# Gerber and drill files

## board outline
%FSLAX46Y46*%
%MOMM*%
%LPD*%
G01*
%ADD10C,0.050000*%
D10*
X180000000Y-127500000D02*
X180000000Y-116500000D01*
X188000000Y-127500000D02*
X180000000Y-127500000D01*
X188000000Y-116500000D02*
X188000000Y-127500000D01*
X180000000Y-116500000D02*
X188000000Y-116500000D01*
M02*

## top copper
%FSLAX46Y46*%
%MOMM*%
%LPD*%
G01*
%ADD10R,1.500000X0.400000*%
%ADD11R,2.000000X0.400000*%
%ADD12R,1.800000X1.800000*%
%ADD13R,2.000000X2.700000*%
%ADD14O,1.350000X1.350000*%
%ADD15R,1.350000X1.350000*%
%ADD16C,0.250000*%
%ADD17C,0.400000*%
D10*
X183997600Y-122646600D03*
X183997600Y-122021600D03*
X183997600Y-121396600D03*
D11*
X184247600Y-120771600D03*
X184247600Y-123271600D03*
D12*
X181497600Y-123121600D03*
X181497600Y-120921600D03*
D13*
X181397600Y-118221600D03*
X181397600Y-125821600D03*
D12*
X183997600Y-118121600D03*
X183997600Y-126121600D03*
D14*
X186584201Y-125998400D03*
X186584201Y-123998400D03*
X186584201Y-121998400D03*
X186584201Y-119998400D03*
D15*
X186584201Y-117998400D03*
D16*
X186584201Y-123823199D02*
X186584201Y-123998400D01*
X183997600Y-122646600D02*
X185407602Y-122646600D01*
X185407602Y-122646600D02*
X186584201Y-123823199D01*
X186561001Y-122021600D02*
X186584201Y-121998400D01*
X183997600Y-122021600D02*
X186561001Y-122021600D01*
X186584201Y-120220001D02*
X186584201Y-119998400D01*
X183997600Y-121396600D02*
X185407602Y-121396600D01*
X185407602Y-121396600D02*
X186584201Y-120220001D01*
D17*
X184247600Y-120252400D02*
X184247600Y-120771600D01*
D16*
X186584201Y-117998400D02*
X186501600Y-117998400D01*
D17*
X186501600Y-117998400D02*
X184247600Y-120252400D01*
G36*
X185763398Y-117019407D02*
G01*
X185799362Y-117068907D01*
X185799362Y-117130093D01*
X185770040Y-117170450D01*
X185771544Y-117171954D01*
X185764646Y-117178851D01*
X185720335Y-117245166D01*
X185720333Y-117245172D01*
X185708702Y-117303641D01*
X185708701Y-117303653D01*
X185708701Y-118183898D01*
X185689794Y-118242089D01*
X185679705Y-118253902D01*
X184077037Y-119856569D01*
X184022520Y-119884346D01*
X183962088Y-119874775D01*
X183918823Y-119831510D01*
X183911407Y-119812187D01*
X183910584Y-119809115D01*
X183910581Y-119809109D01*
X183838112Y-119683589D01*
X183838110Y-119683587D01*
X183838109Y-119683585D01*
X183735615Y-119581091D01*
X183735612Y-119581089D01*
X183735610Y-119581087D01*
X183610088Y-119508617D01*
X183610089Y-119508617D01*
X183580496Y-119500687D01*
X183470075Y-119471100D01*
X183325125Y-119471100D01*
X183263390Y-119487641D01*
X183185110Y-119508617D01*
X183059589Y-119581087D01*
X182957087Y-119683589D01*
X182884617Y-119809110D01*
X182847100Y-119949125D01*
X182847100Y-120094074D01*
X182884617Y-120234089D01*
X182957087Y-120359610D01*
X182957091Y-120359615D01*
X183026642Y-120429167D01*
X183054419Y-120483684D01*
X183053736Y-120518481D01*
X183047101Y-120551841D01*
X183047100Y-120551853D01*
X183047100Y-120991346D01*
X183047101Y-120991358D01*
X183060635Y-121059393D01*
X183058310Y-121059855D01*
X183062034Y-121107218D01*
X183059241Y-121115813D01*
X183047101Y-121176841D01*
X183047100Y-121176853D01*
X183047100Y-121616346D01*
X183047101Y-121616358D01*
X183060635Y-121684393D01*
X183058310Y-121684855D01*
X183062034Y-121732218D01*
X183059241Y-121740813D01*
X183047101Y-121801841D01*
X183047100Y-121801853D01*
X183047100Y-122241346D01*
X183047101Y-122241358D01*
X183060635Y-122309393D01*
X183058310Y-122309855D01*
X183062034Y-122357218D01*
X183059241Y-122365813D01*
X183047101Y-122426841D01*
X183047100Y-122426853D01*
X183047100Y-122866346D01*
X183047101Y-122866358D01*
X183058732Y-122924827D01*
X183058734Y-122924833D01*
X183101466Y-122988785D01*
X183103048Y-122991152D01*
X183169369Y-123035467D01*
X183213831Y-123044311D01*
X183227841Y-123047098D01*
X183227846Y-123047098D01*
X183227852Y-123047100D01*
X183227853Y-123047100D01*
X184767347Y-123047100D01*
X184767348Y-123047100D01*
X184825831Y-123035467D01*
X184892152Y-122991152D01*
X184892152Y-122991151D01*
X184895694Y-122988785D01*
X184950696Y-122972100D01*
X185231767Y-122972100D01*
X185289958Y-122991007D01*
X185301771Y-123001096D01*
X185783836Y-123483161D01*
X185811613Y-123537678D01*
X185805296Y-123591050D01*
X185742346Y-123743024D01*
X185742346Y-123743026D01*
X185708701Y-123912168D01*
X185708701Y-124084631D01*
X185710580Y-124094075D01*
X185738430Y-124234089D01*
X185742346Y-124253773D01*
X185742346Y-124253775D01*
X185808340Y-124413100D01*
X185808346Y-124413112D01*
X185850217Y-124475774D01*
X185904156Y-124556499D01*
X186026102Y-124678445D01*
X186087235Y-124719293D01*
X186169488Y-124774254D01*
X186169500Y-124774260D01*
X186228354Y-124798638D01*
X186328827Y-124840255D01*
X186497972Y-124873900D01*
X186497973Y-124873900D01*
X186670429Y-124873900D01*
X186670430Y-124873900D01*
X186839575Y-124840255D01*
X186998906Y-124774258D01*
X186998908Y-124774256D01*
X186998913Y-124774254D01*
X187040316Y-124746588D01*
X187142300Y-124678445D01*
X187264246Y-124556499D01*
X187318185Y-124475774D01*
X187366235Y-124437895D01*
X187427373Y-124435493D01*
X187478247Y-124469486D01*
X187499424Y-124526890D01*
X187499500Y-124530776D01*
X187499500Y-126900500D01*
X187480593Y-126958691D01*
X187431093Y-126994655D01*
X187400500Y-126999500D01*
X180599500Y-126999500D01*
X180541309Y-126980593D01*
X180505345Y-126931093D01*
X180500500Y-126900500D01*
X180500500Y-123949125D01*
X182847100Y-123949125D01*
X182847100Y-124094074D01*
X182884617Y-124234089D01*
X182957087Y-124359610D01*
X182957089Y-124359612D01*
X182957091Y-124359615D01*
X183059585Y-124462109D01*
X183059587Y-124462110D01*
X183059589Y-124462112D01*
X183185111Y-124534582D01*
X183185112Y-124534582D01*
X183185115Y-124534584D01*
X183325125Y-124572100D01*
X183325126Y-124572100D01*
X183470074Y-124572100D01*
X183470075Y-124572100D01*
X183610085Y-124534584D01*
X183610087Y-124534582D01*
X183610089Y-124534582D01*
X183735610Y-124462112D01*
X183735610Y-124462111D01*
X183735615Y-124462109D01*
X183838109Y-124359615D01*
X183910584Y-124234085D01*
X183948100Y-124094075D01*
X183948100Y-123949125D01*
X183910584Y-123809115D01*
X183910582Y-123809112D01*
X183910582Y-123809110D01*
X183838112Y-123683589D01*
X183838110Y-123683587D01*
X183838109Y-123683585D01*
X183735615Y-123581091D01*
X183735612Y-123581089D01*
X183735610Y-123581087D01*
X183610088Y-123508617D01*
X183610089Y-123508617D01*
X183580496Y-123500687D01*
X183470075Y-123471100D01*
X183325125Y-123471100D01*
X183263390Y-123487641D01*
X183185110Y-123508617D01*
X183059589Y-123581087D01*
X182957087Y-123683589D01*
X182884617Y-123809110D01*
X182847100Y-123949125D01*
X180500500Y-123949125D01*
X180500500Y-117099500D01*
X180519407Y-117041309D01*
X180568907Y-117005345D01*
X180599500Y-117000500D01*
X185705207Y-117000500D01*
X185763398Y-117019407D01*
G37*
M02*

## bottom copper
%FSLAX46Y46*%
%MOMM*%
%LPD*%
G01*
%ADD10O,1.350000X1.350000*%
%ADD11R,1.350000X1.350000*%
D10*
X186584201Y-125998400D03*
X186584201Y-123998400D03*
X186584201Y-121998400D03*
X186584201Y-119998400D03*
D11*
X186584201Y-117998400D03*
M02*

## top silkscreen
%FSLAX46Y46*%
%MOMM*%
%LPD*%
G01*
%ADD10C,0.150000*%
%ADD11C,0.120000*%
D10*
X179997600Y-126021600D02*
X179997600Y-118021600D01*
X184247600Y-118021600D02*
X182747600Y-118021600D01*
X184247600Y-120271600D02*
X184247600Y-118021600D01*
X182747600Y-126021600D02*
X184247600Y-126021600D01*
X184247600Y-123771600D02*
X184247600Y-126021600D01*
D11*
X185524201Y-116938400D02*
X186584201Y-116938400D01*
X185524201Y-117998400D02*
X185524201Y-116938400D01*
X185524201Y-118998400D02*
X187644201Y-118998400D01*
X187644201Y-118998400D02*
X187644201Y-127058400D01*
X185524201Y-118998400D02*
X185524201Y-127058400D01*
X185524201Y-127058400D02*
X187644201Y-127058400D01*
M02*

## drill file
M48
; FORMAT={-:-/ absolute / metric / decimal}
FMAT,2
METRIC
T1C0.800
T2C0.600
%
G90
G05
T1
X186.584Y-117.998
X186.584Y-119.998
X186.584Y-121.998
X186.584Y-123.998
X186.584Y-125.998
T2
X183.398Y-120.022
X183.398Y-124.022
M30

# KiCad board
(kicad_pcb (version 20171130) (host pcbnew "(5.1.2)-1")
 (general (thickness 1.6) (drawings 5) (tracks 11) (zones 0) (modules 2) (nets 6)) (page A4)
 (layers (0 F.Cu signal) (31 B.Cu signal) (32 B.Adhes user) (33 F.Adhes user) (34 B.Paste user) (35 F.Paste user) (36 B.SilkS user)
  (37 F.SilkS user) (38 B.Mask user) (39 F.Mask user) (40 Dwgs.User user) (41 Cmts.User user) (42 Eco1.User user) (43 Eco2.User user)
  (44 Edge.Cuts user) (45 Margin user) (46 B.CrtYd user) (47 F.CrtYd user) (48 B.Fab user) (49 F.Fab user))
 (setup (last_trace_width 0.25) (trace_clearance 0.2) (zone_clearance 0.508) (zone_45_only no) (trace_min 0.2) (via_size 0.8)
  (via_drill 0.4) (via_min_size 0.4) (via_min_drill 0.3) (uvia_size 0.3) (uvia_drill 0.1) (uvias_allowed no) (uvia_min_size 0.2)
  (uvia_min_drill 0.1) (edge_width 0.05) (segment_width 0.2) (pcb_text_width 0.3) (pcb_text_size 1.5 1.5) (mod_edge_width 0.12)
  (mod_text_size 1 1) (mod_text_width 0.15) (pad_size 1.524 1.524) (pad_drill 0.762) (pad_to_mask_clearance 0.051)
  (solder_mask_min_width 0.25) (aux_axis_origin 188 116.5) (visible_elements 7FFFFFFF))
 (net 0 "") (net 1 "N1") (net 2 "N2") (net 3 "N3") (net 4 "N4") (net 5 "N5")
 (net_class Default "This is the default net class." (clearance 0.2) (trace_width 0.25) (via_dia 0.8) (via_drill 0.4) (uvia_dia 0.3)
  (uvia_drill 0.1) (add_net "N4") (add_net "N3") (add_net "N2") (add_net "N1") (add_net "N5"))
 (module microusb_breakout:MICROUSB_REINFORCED (layer F.Cu) (at 183.9976 122.0216 90) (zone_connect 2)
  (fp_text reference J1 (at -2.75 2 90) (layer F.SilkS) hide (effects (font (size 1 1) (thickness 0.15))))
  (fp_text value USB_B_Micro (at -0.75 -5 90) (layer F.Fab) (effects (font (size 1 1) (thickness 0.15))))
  (fp_line (start -4 -4) (end 4 -4) (layer F.SilkS) (width 0.15))
  (fp_line (start 4 0.25) (end 4 -1.25) (layer F.SilkS) (width 0.15))
  (fp_line (start 1.75 0.25) (end 4 0.25) (layer F.SilkS) (width 0.15))
  (fp_line (start -4 -1.25) (end -4 0.25) (layer F.SilkS) (width 0.15))
  (fp_line (start -1.75 0.25) (end -4 0.25) (layer F.SilkS) (width 0.15))
  (pad 4 smd rect (at -0.625 0 90) (size 0.4 1.5) (layers F.Cu F.Paste F.Mask) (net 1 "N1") (zone_connect 2))
  (pad 3 smd rect (at 0 0 90) (size 0.4 1.5) (layers F.Cu F.Paste F.Mask) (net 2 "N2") (zone_connect 2))
  (pad 2 smd rect (at 0.625 0 90) (size 0.4 1.5) (layers F.Cu F.Paste F.Mask) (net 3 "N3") (zone_connect 2))
  (pad 1 smd rect (at 1.25 0.25 90) (size 0.4 2) (layers F.Cu F.Paste F.Mask) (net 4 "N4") (zone_connect 2))
  (pad 5 smd rect (at -1.25 0.25 90) (size 0.4 2) (layers F.Cu F.Paste F.Mask) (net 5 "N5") (zone_connect 2))
  (pad 6 smd rect (at -1.1 -2.5 90) (size 1.8 1.8) (layers F.Cu F.Paste F.Mask) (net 5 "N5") (zone_connect 2))
  (pad 6 smd rect (at 1.1 -2.5 90) (size 1.8 1.8) (layers F.Cu F.Paste F.Mask) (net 5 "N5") (zone_connect 2))
  (pad 6 smd rect (at 3.8 -2.6 90) (size 2.7 2) (layers F.Cu F.Paste F.Mask) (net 5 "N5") (zone_connect 2))
  (pad 6 smd rect (at -3.8 -2.6 90) (size 2.7 2) (layers F.Cu F.Paste F.Mask) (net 5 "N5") (zone_connect 2))
  (pad "" np_thru_hole circle (at 2 -0.6 90) (size 0.6 0.6) (drill 0.6) (layers *.Cu *.Mask) (zone_connect 2))
  (pad "" np_thru_hole circle (at -2 -0.6 90) (size 0.6 0.6) (drill 0.6) (layers *.Cu *.Mask) (zone_connect 2))
  (pad 6 smd rect (at 3.9 0 90) (size 1.8 1.8) (layers F.Cu F.Paste F.Mask) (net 5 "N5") (zone_connect 2))
  (pad 6 smd rect (at -4.1 0 90) (size 1.8 1.8) (layers F.Cu F.Paste F.Mask) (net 5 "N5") (zone_connect 2)))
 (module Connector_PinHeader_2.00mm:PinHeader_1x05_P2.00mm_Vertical (layer F.Cu) (at 186.584201 117.9984)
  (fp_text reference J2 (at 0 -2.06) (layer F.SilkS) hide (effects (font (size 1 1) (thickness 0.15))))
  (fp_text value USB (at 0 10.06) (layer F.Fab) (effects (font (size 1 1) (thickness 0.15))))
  (fp_line (start -1.06 -1.06) (end 0 -1.06) (layer F.SilkS) (width 0.12))
  (fp_line (start -1.06 0) (end -1.06 -1.06) (layer F.SilkS) (width 0.12))
  (fp_line (start -1.06 1) (end 1.06 1) (layer F.SilkS) (width 0.12))
  (fp_line (start 1.06 1) (end 1.06 9.06) (layer F.SilkS) (width 0.12))
  (fp_line (start -1.06 1) (end -1.06 9.06) (layer F.SilkS) (width 0.12))
  (fp_line (start -1.06 9.06) (end 1.06 9.06) (layer F.SilkS) (width 0.12))
  (pad 5 thru_hole oval (at 0 8) (size 1.35 1.35) (drill 0.8) (layers *.Cu *.Mask) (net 5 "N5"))
  (pad 4 thru_hole oval (at 0 6) (size 1.35 1.35) (drill 0.8) (layers *.Cu *.Mask) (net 1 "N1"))
  (pad 3 thru_hole oval (at 0 4) (size 1.35 1.35) (drill 0.8) (layers *.Cu *.Mask) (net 2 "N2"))
  (pad 2 thru_hole oval (at 0 2) (size 1.35 1.35) (drill 0.8) (layers *.Cu *.Mask) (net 3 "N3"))
  (pad 1 thru_hole rect (at 0 0) (size 1.35 1.35) (drill 0.8) (layers *.Cu *.Mask) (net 4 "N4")))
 (gr_line (start 180 127.5) (end 180 116.5) (layer Edge.Cuts) (width 0.05))
 (gr_line (start 188 127.5) (end 180 127.5) (layer Edge.Cuts) (width 0.05))
 (gr_line (start 188 116.5) (end 188 127.5) (layer Edge.Cuts) (width 0.05))
 (gr_line (start 180 116.5) (end 188 116.5) (layer Edge.Cuts) (width 0.05))
 (segment (start 186.584201 123.823199) (end 186.584201 123.9984) (width 0.25) (layer F.Cu) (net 1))
 (segment (start 183.9976 122.6466) (end 185.407602 122.6466) (width 0.25) (layer F.Cu) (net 1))
 (segment (start 185.407602 122.6466) (end 186.584201 123.823199) (width 0.25) (layer F.Cu) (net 1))
 (segment (start 186.561001 122.0216) (end 186.584201 121.9984) (width 0.25) (layer F.Cu) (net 2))
 (segment (start 183.9976 122.0216) (end 186.561001 122.0216) (width 0.25) (layer F.Cu) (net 2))
 (segment (start 186.584201 120.220001) (end 186.584201 119.9984) (width 0.25) (layer F.Cu) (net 3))
 (segment (start 183.9976 121.3966) (end 185.407602 121.3966) (width 0.25) (layer F.Cu) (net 3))
 (segment (start 185.407602 121.3966) (end 186.584201 120.220001) (width 0.25) (layer F.Cu) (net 3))
 (segment (start 184.2476 120.2524) (end 184.2476 120.7716) (width 0.4) (layer F.Cu) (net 4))
 (segment (start 186.584201 117.9984) (end 186.5016 117.9984) (width 0.25) (layer F.Cu) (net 4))
 (segment (start 186.5016 117.9984) (end 184.2476 120.2524) (width 0.4) (layer F.Cu) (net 4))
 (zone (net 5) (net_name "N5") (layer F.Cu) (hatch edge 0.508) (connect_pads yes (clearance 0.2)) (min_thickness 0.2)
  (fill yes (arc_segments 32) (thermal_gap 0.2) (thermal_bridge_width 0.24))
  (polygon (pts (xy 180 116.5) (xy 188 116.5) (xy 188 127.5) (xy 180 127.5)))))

